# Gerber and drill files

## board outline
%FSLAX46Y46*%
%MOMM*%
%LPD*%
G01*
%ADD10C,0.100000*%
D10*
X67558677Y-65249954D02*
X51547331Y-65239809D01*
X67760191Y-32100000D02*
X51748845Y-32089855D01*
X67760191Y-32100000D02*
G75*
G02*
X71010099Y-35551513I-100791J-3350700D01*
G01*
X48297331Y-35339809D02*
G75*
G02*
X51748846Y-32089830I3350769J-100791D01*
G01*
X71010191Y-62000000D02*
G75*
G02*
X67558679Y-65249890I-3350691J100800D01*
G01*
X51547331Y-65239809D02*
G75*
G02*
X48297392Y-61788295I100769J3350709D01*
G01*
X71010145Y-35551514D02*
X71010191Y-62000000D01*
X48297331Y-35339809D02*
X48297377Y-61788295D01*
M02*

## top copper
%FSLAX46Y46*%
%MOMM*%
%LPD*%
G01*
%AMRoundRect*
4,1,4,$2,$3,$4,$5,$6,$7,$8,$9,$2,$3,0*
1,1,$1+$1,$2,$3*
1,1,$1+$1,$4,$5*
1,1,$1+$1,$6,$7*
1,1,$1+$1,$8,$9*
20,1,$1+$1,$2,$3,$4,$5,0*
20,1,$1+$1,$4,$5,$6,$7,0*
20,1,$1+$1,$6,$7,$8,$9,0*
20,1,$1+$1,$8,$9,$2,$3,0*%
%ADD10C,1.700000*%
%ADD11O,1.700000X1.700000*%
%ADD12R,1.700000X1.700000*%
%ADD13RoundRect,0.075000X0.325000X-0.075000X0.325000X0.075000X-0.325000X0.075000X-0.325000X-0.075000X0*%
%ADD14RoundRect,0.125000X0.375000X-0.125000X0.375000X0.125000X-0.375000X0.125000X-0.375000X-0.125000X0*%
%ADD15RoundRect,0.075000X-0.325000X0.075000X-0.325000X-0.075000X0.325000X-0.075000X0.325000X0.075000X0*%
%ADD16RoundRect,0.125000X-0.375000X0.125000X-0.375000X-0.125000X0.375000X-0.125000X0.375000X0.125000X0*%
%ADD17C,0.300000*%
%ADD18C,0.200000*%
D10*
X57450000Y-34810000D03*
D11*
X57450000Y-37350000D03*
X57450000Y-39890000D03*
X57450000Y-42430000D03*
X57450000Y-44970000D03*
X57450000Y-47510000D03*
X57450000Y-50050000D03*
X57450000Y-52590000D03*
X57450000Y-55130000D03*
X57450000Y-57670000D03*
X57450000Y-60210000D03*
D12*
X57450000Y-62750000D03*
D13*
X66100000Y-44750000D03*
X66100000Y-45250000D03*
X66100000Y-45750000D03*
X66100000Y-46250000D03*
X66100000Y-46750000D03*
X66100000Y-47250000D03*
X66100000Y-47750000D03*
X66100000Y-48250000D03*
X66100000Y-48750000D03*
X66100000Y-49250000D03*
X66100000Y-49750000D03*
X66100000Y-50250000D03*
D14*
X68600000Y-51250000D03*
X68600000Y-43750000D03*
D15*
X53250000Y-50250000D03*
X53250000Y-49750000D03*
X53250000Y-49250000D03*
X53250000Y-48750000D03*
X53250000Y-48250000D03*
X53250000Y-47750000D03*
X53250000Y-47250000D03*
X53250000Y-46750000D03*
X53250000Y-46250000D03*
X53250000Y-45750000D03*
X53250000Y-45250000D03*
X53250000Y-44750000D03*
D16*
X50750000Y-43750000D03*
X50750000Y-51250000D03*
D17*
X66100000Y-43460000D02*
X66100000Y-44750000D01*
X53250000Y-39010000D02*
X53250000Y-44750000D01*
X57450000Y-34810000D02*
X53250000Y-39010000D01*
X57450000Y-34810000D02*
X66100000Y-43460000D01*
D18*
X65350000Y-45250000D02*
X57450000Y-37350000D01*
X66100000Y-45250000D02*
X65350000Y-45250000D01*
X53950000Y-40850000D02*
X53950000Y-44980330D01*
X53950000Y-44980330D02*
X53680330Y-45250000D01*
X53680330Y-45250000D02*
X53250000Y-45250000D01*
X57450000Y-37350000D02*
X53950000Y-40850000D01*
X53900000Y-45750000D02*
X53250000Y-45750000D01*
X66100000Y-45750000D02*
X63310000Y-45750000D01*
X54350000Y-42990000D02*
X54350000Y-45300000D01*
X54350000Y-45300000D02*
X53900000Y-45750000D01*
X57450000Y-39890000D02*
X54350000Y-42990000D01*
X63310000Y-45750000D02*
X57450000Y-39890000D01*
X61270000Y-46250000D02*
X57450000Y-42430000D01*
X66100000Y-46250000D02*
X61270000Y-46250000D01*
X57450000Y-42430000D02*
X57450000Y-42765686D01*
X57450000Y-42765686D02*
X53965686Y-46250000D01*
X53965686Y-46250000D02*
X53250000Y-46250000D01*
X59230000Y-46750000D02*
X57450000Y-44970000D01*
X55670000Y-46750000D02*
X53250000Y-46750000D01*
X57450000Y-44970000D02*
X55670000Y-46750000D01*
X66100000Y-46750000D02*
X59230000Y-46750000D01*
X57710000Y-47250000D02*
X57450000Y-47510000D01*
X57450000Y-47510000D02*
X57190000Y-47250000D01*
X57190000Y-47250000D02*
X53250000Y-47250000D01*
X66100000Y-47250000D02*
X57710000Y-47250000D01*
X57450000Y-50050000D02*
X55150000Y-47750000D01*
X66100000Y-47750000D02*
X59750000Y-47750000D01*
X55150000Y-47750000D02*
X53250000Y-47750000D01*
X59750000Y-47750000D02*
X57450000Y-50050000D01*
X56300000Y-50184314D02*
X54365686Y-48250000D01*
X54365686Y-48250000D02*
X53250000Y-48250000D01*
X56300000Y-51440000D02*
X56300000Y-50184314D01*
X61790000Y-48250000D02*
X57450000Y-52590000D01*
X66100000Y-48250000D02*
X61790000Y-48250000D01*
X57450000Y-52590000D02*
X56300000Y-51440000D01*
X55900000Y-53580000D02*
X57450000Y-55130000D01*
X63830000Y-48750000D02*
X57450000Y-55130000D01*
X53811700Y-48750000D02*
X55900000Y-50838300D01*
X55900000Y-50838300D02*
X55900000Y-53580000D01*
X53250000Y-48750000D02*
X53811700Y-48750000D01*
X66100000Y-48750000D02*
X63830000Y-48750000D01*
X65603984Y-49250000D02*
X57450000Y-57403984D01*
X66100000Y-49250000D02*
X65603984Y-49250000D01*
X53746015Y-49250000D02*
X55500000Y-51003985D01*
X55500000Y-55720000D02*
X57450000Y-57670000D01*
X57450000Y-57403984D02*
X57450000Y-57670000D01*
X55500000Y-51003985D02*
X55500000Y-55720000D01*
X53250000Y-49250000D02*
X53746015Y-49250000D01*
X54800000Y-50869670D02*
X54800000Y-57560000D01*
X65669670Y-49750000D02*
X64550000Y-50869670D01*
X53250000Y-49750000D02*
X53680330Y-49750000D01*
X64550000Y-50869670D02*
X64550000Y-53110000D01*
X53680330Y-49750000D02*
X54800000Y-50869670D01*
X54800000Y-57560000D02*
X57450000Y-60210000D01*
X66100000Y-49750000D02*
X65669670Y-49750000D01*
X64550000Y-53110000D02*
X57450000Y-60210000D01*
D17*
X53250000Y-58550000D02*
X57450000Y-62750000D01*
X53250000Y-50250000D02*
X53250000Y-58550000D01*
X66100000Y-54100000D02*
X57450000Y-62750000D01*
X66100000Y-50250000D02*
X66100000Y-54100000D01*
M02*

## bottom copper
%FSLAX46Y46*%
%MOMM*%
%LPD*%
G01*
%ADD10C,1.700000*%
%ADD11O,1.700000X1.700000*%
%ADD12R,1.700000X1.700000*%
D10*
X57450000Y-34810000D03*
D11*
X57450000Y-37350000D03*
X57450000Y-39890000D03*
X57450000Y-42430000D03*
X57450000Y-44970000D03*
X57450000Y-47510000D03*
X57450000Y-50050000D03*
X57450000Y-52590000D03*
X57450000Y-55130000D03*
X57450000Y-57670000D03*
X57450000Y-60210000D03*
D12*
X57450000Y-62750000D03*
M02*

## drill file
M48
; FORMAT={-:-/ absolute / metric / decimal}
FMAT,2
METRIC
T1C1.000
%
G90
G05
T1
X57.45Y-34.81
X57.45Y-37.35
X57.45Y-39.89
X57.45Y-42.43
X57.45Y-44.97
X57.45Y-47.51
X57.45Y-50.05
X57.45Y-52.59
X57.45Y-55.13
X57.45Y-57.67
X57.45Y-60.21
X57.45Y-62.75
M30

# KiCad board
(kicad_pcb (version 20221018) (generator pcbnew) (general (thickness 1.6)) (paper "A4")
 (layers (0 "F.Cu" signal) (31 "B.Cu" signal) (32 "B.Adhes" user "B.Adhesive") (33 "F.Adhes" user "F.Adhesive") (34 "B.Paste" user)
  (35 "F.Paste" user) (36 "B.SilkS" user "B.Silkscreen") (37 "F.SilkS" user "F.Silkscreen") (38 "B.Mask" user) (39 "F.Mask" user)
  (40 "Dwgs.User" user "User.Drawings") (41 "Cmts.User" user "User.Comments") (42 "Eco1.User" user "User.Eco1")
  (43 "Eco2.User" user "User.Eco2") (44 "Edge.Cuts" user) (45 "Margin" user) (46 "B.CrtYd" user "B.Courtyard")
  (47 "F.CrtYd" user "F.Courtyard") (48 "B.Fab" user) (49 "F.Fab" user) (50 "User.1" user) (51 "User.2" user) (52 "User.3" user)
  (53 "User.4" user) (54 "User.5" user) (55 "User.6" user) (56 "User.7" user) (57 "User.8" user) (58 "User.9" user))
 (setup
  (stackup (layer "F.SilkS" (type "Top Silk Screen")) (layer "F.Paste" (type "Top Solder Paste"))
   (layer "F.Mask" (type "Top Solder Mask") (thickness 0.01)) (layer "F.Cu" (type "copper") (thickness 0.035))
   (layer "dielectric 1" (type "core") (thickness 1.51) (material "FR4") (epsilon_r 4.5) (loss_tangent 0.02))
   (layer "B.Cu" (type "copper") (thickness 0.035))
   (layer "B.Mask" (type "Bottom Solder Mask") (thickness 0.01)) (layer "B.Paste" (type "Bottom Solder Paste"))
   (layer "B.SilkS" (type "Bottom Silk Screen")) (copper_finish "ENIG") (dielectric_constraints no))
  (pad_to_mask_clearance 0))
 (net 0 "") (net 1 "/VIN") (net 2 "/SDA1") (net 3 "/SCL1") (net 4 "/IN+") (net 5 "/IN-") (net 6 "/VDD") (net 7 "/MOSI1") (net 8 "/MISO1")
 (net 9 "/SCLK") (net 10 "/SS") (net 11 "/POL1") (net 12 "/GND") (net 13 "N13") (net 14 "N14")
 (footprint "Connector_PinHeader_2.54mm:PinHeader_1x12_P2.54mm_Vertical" (layer "F.Cu") (at 57.45 34.81)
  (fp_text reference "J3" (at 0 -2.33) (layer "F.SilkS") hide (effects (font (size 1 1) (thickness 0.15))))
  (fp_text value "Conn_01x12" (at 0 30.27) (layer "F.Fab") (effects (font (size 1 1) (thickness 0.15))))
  (pad "1" thru_hole circle (at 0 0) (size 1.7 1.7) (drill 1) (layers "*.Cu" "*.Mask") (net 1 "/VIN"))
  (pad "2" thru_hole oval (at 0 2.54) (size 1.7 1.7) (drill 1) (layers "*.Cu" "*.Mask") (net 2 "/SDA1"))
  (pad "3" thru_hole oval (at 0 5.08) (size 1.7 1.7) (drill 1) (layers "*.Cu" "*.Mask") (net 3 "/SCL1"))
  (pad "4" thru_hole oval (at 0 7.62) (size 1.7 1.7) (drill 1) (layers "*.Cu" "*.Mask") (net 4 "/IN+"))
  (pad "5" thru_hole oval (at 0 10.16) (size 1.7 1.7) (drill 1) (layers "*.Cu" "*.Mask") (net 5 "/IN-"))
  (pad "6" thru_hole oval (at 0 12.7) (size 1.7 1.7) (drill 1) (layers "*.Cu" "*.Mask") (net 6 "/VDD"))
  (pad "7" thru_hole oval (at 0 15.24) (size 1.7 1.7) (drill 1) (layers "*.Cu" "*.Mask") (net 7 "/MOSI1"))
  (pad "8" thru_hole oval (at 0 17.78) (size 1.7 1.7) (drill 1) (layers "*.Cu" "*.Mask") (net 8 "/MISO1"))
  (pad "9" thru_hole oval (at 0 20.32) (size 1.7 1.7) (drill 1) (layers "*.Cu" "*.Mask") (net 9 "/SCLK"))
  (pad "10" thru_hole oval (at 0 22.86) (size 1.7 1.7) (drill 1) (layers "*.Cu" "*.Mask") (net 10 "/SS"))
  (pad "11" thru_hole oval (at 0 25.4) (size 1.7 1.7) (drill 1) (layers "*.Cu" "*.Mask") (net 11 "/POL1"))
  (pad "12" thru_hole rect (at 0 27.94) (size 1.7 1.7) (drill 1) (layers "*.Cu" "*.Mask") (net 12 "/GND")))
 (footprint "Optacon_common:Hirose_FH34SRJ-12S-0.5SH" (layer "F.Cu") (at 67.2 47.5 90)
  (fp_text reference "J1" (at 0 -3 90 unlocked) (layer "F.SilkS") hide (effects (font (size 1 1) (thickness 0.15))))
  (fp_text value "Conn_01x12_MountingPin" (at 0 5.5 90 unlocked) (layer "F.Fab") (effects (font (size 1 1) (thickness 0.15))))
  (pad "" smd roundrect (at -2.75 -1.1 90) (size 0.4 0.8) (layers "F.Paste") (roundrect_rratio 0.25) (solder_paste_margin -0.05))
  (pad "" smd roundrect (at -2.25 -1.1 90) (size 0.4 0.8) (layers "F.Paste") (roundrect_rratio 0.25) (solder_paste_margin -0.05))
  (pad "" smd roundrect (at -1.75 -1.1 90) (size 0.4 0.8) (layers "F.Paste") (roundrect_rratio 0.25) (solder_paste_margin -0.05))
  (pad "" smd roundrect (at -1.25 -1.1 90) (size 0.4 0.8) (layers "F.Paste") (roundrect_rratio 0.25) (solder_paste_margin -0.05))
  (pad "" smd roundrect (at -0.75 -1.1 90) (size 0.4 0.8) (layers "F.Paste") (roundrect_rratio 0.25) (solder_paste_margin -0.05))
  (pad "" smd roundrect (at -0.25 -1.1 90) (size 0.4 0.8) (layers "F.Paste") (roundrect_rratio 0.25) (solder_paste_margin -0.05))
  (pad "" smd roundrect (at 0.25 -1.1 90) (size 0.4 0.8) (layers "F.Paste") (roundrect_rratio 0.25) (solder_paste_margin -0.05))
  (pad "" smd roundrect (at 0.75 -1.1 90) (size 0.4 0.8) (layers "F.Paste") (roundrect_rratio 0.25) (solder_paste_margin -0.05))
  (pad "" smd roundrect (at 1.25 -1.1 90) (size 0.4 0.8) (layers "F.Paste") (roundrect_rratio 0.25) (solder_paste_margin -0.05))
  (pad "" smd roundrect (at 1.75 -1.1 90) (size 0.4 0.8) (layers "F.Paste") (roundrect_rratio 0.25) (solder_paste_margin -0.05))
  (pad "" smd roundrect (at 2.25 -1.1 90) (size 0.4 0.8) (layers "F.Paste") (roundrect_rratio 0.25) (solder_paste_margin -0.05))
  (pad "" smd roundrect (at 2.75 -1.1 90) (size 0.4 0.8) (layers "F.Paste") (roundrect_rratio 0.25) (solder_paste_margin -0.05))
  (pad "1" smd roundrect (at 2.75 -1.1 90) (size 0.3 0.8) (layers "F.Cu" "F.Paste" "F.Mask") (roundrect_rratio 0.25) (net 1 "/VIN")
   (solder_paste_margin -0.05))
  (pad "2" smd roundrect (at 2.25 -1.1 90) (size 0.3 0.8) (layers "F.Cu" "F.Paste" "F.Mask") (roundrect_rratio 0.25) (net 2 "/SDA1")
   (solder_paste_margin -0.05))
  (pad "3" smd roundrect (at 1.75 -1.1 90) (size 0.3 0.8) (layers "F.Cu" "F.Paste" "F.Mask") (roundrect_rratio 0.25) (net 3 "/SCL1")
   (solder_paste_margin -0.05))
  (pad "4" smd roundrect (at 1.25 -1.1 90) (size 0.3 0.8) (layers "F.Cu" "F.Paste" "F.Mask") (roundrect_rratio 0.25) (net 4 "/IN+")
   (solder_paste_margin -0.05))
  (pad "5" smd roundrect (at 0.75 -1.1 90) (size 0.3 0.8) (layers "F.Cu" "F.Paste" "F.Mask") (roundrect_rratio 0.25) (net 5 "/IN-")
   (solder_paste_margin -0.05))
  (pad "6" smd roundrect (at 0.25 -1.1 90) (size 0.3 0.8) (layers "F.Cu" "F.Paste" "F.Mask") (roundrect_rratio 0.25) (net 6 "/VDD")
   (solder_paste_margin -0.05))
  (pad "7" smd roundrect (at -0.25 -1.1 90) (size 0.3 0.8) (layers "F.Cu" "F.Paste" "F.Mask") (roundrect_rratio 0.25) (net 7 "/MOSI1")
   (solder_paste_margin -0.05))
  (pad "8" smd roundrect (at -0.75 -1.1 90) (size 0.3 0.8) (layers "F.Cu" "F.Paste" "F.Mask") (roundrect_rratio 0.25) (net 8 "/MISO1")
   (solder_paste_margin -0.05))
  (pad "9" smd roundrect (at -1.25 -1.1 90) (size 0.3 0.8) (layers "F.Cu" "F.Paste" "F.Mask") (roundrect_rratio 0.25) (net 9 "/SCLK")
   (solder_paste_margin -0.05))
  (pad "10" smd roundrect (at -1.75 -1.1 90) (size 0.3 0.8) (layers "F.Cu" "F.Paste" "F.Mask") (roundrect_rratio 0.25) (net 10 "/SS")
   (solder_paste_margin -0.05))
  (pad "11" smd roundrect (at -2.25 -1.1 90) (size 0.3 0.8) (layers "F.Cu" "F.Paste" "F.Mask") (roundrect_rratio 0.25) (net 11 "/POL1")
   (solder_paste_margin -0.05))
  (pad "12" smd roundrect (at -2.75 -1.1 90) (size 0.3 0.8) (layers "F.Cu" "F.Mask") (roundrect_rratio 0.25) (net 12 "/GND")
   (solder_paste_margin -0.05))
  (pad "MP" smd roundrect (at -3.75 1.4 90) (size 0.5 1) (layers "F.Cu" "F.Paste" "F.Mask") (roundrect_rratio 0.25) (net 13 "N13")
   (solder_paste_margin -0.05))
  (pad "MP" smd roundrect (at 3.75 1.4 90) (size 0.5 1) (layers "F.Cu" "F.Paste" "F.Mask") (roundrect_rratio 0.25) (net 13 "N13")
   (solder_paste_margin -0.05)))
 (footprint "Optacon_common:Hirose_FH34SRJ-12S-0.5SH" (layer "F.Cu") (at 52.15 47.5 -90)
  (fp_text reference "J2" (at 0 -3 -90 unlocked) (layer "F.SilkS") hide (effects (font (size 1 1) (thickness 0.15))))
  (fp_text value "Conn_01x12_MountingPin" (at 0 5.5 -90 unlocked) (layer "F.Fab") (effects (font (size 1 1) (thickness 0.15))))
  (pad "" smd roundrect (at -2.75 -1.1 270) (size 0.4 0.8) (layers "F.Paste") (roundrect_rratio 0.25) (solder_paste_margin -0.05))
  (pad "" smd roundrect (at -2.25 -1.1 270) (size 0.4 0.8) (layers "F.Paste") (roundrect_rratio 0.25) (solder_paste_margin -0.05))
  (pad "" smd roundrect (at -1.75 -1.1 270) (size 0.4 0.8) (layers "F.Paste") (roundrect_rratio 0.25) (solder_paste_margin -0.05))
  (pad "" smd roundrect (at -1.25 -1.1 270) (size 0.4 0.8) (layers "F.Paste") (roundrect_rratio 0.25) (solder_paste_margin -0.05))
  (pad "" smd roundrect (at -0.75 -1.1 270) (size 0.4 0.8) (layers "F.Paste") (roundrect_rratio 0.25) (solder_paste_margin -0.05))
  (pad "" smd roundrect (at -0.25 -1.1 270) (size 0.4 0.8) (layers "F.Paste") (roundrect_rratio 0.25) (solder_paste_margin -0.05))
  (pad "" smd roundrect (at 0.25 -1.1 270) (size 0.4 0.8) (layers "F.Paste") (roundrect_rratio 0.25) (solder_paste_margin -0.05))
  (pad "" smd roundrect (at 0.75 -1.1 270) (size 0.4 0.8) (layers "F.Paste") (roundrect_rratio 0.25) (solder_paste_margin -0.05))
  (pad "" smd roundrect (at 1.25 -1.1 270) (size 0.4 0.8) (layers "F.Paste") (roundrect_rratio 0.25) (solder_paste_margin -0.05))
  (pad "" smd roundrect (at 1.75 -1.1 270) (size 0.4 0.8) (layers "F.Paste") (roundrect_rratio 0.25) (solder_paste_margin -0.05))
  (pad "" smd roundrect (at 2.25 -1.1 270) (size 0.4 0.8) (layers "F.Paste") (roundrect_rratio 0.25) (solder_paste_margin -0.05))
  (pad "" smd roundrect (at 2.75 -1.1 270) (size 0.4 0.8) (layers "F.Paste") (roundrect_rratio 0.25) (solder_paste_margin -0.05))
  (pad "1" smd roundrect (at 2.75 -1.1 270) (size 0.3 0.8) (layers "F.Cu" "F.Paste" "F.Mask") (roundrect_rratio 0.25) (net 12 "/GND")
   (solder_paste_margin -0.05))
  (pad "2" smd roundrect (at 2.25 -1.1 270) (size 0.3 0.8) (layers "F.Cu" "F.Paste" "F.Mask") (roundrect_rratio 0.25) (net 11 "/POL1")
   (solder_paste_margin -0.05))
  (pad "3" smd roundrect (at 1.75 -1.1 270) (size 0.3 0.8) (layers "F.Cu" "F.Paste" "F.Mask") (roundrect_rratio 0.25) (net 10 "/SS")
   (solder_paste_margin -0.05))
  (pad "4" smd roundrect (at 1.25 -1.1 270) (size 0.3 0.8) (layers "F.Cu" "F.Paste" "F.Mask") (roundrect_rratio 0.25) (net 9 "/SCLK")
   (solder_paste_margin -0.05))
  (pad "5" smd roundrect (at 0.75 -1.1 270) (size 0.3 0.8) (layers "F.Cu" "F.Paste" "F.Mask") (roundrect_rratio 0.25) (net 8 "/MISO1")
   (solder_paste_margin -0.05))
  (pad "6" smd roundrect (at 0.25 -1.1 270) (size 0.3 0.8) (layers "F.Cu" "F.Paste" "F.Mask") (roundrect_rratio 0.25) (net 7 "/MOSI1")
   (solder_paste_margin -0.05))
  (pad "7" smd roundrect (at -0.25 -1.1 270) (size 0.3 0.8) (layers "F.Cu" "F.Paste" "F.Mask") (roundrect_rratio 0.25) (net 6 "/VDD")
   (solder_paste_margin -0.05))
  (pad "8" smd roundrect (at -0.75 -1.1 270) (size 0.3 0.8) (layers "F.Cu" "F.Paste" "F.Mask") (roundrect_rratio 0.25) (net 5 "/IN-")
   (solder_paste_margin -0.05))
  (pad "9" smd roundrect (at -1.25 -1.1 270) (size 0.3 0.8) (layers "F.Cu" "F.Paste" "F.Mask") (roundrect_rratio 0.25) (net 4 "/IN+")
   (solder_paste_margin -0.05))
  (pad "10" smd roundrect (at -1.75 -1.1 270) (size 0.3 0.8) (layers "F.Cu" "F.Paste" "F.Mask") (roundrect_rratio 0.25) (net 3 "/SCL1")
   (solder_paste_margin -0.05))
  (pad "11" smd roundrect (at -2.25 -1.1 270) (size 0.3 0.8) (layers "F.Cu" "F.Paste" "F.Mask") (roundrect_rratio 0.25) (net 2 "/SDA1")
   (solder_paste_margin -0.05))
  (pad "12" smd roundrect (at -2.75 -1.1 270) (size 0.3 0.8) (layers "F.Cu" "F.Mask") (roundrect_rratio 0.25) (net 1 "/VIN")
   (solder_paste_margin -0.05))
  (pad "MP" smd roundrect (at -3.75 1.4 270) (size 0.5 1) (layers "F.Cu" "F.Paste" "F.Mask") (roundrect_rratio 0.25) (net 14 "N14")
   (solder_paste_margin -0.05))
  (pad "MP" smd roundrect (at 3.75 1.4 270) (size 0.5 1) (layers "F.Cu" "F.Paste" "F.Mask") (roundrect_rratio 0.25) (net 14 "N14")
   (solder_paste_margin -0.05)))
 (gr_line (start 67.558677 65.249954) (end 51.547331 65.239809) (stroke (width 0.1) (type default)) (layer "Edge.Cuts"))
 (gr_line (start 67.760191 32.1) (end 51.748845 32.089855) (stroke (width 0.1) (type default)) (layer "Edge.Cuts"))
 (gr_arc (start 67.760191 32.1) (mid 70.1 33.152669) (end 71.010145 35.551514) (stroke (width 0.1) (type default)) (layer "Edge.Cuts"))
 (gr_arc (start 48.297331 35.339809) (mid 49.35 33) (end 51.748845 32.089855) (stroke (width 0.1) (type default)) (layer "Edge.Cuts"))
 (gr_arc (start 71.010191 62) (mid 69.957522 64.339809) (end 67.558677 65.249954) (stroke (width 0.1) (type default)) (layer "Edge.Cuts"))
 (gr_arc (start 51.547331 65.239809) (mid 49.207522 64.18714) (end 48.297377 61.788295) (stroke (width 0.1) (type default))
  (layer "Edge.Cuts"))
 (gr_line (start 71.010145 35.551514) (end 71.010191 62) (stroke (width 0.1) (type default)) (layer "Edge.Cuts"))
 (gr_line (start 48.297331 35.339809) (end 48.297377 61.788295) (stroke (width 0.1) (type default)) (layer "Edge.Cuts"))
 (segment (start 66.1 43.46) (end 66.1 44.75) (width 0.3) (layer "F.Cu") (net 1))
 (segment (start 53.25 39.01) (end 53.25 44.75) (width 0.3) (layer "F.Cu") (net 1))
 (segment (start 57.45 34.81) (end 53.25 39.01) (width 0.3) (layer "F.Cu") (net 1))
 (segment (start 57.45 34.81) (end 66.1 43.46) (width 0.3) (layer "F.Cu") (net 1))
 (segment (start 65.35 45.25) (end 57.45 37.35) (width 0.2) (layer "F.Cu") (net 2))
 (segment (start 66.1 45.25) (end 65.35 45.25) (width 0.2) (layer "F.Cu") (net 2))
 (segment (start 53.95 40.85) (end 53.95 44.98033) (width 0.2) (layer "F.Cu") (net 2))
 (segment (start 53.95 44.98033) (end 53.68033 45.25) (width 0.2) (layer "F.Cu") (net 2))
 (segment (start 53.68033 45.25) (end 53.25 45.25) (width 0.2) (layer "F.Cu") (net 2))
 (segment (start 57.45 37.35) (end 53.95 40.85) (width 0.2) (layer "F.Cu") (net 2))
 (segment (start 53.9 45.75) (end 53.25 45.75) (width 0.2) (layer "F.Cu") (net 3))
 (segment (start 66.1 45.75) (end 63.31 45.75) (width 0.2) (layer "F.Cu") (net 3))
 (segment (start 54.35 42.99) (end 54.35 45.3) (width 0.2) (layer "F.Cu") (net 3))
 (segment (start 54.35 45.3) (end 53.9 45.75) (width 0.2) (layer "F.Cu") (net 3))
 (segment (start 57.45 39.89) (end 54.35 42.99) (width 0.2) (layer "F.Cu") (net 3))
 (segment (start 63.31 45.75) (end 57.45 39.89) (width 0.2) (layer "F.Cu") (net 3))
 (segment (start 61.27 46.25) (end 57.45 42.43) (width 0.2) (layer "F.Cu") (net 4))
 (segment (start 66.1 46.25) (end 61.27 46.25) (width 0.2) (layer "F.Cu") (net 4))
 (segment (start 57.45 42.43) (end 57.45 42.765686) (width 0.2) (layer "F.Cu") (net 4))
 (segment (start 57.45 42.765686) (end 53.965686 46.25) (width 0.2) (layer "F.Cu") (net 4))
 (segment (start 53.965686 46.25) (end 53.25 46.25) (width 0.2) (layer "F.Cu") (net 4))
 (segment (start 59.23 46.75) (end 57.45 44.97) (width 0.2) (layer "F.Cu") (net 5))
 (segment (start 55.67 46.75) (end 53.25 46.75) (width 0.2) (layer "F.Cu") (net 5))
 (segment (start 57.45 44.97) (end 55.67 46.75) (width 0.2) (layer "F.Cu") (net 5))
 (segment (start 66.1 46.75) (end 59.23 46.75) (width 0.2) (layer "F.Cu") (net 5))
 (segment (start 57.71 47.25) (end 57.45 47.51) (width 0.2) (layer "F.Cu") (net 6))
 (segment (start 57.45 47.51) (end 57.19 47.25) (width 0.2) (layer "F.Cu") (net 6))
 (segment (start 57.19 47.25) (end 53.25 47.25) (width 0.2) (layer "F.Cu") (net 6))
 (segment (start 66.1 47.25) (end 57.71 47.25) (width 0.2) (layer "F.Cu") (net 6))
 (segment (start 57.45 50.05) (end 55.15 47.75) (width 0.2) (layer "F.Cu") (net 7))
 (segment (start 66.1 47.75) (end 59.75 47.75) (width 0.2) (layer "F.Cu") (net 7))
 (segment (start 55.15 47.75) (end 53.25 47.75) (width 0.2) (layer "F.Cu") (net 7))
 (segment (start 59.75 47.75) (end 57.45 50.05) (width 0.2) (layer "F.Cu") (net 7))
 (segment (start 56.3 50.184314) (end 54.365686 48.25) (width 0.2) (layer "F.Cu") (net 8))
 (segment (start 54.365686 48.25) (end 53.25 48.25) (width 0.2) (layer "F.Cu") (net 8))
 (segment (start 56.3 51.44) (end 56.3 50.184314) (width 0.2) (layer "F.Cu") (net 8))
 (segment (start 61.79 48.25) (end 57.45 52.59) (width 0.2) (layer "F.Cu") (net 8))
 (segment (start 66.1 48.25) (end 61.79 48.25) (width 0.2) (layer "F.Cu") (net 8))
 (segment (start 57.45 52.59) (end 56.3 51.44) (width 0.2) (layer "F.Cu") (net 8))
 (segment (start 55.9 53.58) (end 57.45 55.13) (width 0.2) (layer "F.Cu") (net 9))
 (segment (start 63.83 48.75) (end 57.45 55.13) (width 0.2) (layer "F.Cu") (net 9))
 (segment (start 53.8117 48.75) (end 55.9 50.8383) (width 0.2) (layer "F.Cu") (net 9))
 (segment (start 55.9 50.8383) (end 55.9 53.58) (width 0.2) (layer "F.Cu") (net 9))
 (segment (start 53.25 48.75) (end 53.8117 48.75) (width 0.2) (layer "F.Cu") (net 9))
 (segment (start 66.1 48.75) (end 63.83 48.75) (width 0.2) (layer "F.Cu") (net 9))
 (segment (start 65.603984 49.25) (end 57.45 57.403984) (width 0.2) (layer "F.Cu") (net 10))
 (segment (start 66.1 49.25) (end 65.603984 49.25) (width 0.2) (layer "F.Cu") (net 10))
 (segment (start 53.746015 49.25) (end 55.5 51.003985) (width 0.2) (layer "F.Cu") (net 10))
 (segment (start 55.5 55.72) (end 57.45 57.67) (width 0.2) (layer "F.Cu") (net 10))
 (segment (start 57.45 57.403984) (end 57.45 57.67) (width 0.2) (layer "F.Cu") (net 10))
 (segment (start 55.5 51.003985) (end 55.5 55.72) (width 0.2) (layer "F.Cu") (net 10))
 (segment (start 53.25 49.25) (end 53.746015 49.25) (width 0.2) (layer "F.Cu") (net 10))
 (segment (start 54.8 50.86967) (end 54.8 57.56) (width 0.2) (layer "F.Cu") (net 11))
 (segment (start 65.66967 49.75) (end 64.55 50.86967) (width 0.2) (layer "F.Cu") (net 11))
 (segment (start 53.25 49.75) (end 53.68033 49.75) (width 0.2) (layer "F.Cu") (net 11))
 (segment (start 64.55 50.86967) (end 64.55 53.11) (width 0.2) (layer "F.Cu") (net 11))
 (segment (start 53.68033 49.75) (end 54.8 50.86967) (width 0.2) (layer "F.Cu") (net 11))
 (segment (start 54.8 57.56) (end 57.45 60.21) (width 0.2) (layer "F.Cu") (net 11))
 (segment (start 66.1 49.75) (end 65.66967 49.75) (width 0.2) (layer "F.Cu") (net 11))
 (segment (start 64.55 53.11) (end 57.45 60.21) (width 0.2) (layer "F.Cu") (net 11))
 (segment (start 53.25 58.55) (end 57.45 62.75) (width 0.3) (layer "F.Cu") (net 12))
 (segment (start 53.25 50.25) (end 53.25 58.55) (width 0.3) (layer "F.Cu") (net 12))
 (segment (start 66.1 54.1) (end 57.45 62.75) (width 0.3) (layer "F.Cu") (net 12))
 (segment (start 66.1 50.25) (end 66.1 54.1) (width 0.3) (layer "F.Cu") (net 12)))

